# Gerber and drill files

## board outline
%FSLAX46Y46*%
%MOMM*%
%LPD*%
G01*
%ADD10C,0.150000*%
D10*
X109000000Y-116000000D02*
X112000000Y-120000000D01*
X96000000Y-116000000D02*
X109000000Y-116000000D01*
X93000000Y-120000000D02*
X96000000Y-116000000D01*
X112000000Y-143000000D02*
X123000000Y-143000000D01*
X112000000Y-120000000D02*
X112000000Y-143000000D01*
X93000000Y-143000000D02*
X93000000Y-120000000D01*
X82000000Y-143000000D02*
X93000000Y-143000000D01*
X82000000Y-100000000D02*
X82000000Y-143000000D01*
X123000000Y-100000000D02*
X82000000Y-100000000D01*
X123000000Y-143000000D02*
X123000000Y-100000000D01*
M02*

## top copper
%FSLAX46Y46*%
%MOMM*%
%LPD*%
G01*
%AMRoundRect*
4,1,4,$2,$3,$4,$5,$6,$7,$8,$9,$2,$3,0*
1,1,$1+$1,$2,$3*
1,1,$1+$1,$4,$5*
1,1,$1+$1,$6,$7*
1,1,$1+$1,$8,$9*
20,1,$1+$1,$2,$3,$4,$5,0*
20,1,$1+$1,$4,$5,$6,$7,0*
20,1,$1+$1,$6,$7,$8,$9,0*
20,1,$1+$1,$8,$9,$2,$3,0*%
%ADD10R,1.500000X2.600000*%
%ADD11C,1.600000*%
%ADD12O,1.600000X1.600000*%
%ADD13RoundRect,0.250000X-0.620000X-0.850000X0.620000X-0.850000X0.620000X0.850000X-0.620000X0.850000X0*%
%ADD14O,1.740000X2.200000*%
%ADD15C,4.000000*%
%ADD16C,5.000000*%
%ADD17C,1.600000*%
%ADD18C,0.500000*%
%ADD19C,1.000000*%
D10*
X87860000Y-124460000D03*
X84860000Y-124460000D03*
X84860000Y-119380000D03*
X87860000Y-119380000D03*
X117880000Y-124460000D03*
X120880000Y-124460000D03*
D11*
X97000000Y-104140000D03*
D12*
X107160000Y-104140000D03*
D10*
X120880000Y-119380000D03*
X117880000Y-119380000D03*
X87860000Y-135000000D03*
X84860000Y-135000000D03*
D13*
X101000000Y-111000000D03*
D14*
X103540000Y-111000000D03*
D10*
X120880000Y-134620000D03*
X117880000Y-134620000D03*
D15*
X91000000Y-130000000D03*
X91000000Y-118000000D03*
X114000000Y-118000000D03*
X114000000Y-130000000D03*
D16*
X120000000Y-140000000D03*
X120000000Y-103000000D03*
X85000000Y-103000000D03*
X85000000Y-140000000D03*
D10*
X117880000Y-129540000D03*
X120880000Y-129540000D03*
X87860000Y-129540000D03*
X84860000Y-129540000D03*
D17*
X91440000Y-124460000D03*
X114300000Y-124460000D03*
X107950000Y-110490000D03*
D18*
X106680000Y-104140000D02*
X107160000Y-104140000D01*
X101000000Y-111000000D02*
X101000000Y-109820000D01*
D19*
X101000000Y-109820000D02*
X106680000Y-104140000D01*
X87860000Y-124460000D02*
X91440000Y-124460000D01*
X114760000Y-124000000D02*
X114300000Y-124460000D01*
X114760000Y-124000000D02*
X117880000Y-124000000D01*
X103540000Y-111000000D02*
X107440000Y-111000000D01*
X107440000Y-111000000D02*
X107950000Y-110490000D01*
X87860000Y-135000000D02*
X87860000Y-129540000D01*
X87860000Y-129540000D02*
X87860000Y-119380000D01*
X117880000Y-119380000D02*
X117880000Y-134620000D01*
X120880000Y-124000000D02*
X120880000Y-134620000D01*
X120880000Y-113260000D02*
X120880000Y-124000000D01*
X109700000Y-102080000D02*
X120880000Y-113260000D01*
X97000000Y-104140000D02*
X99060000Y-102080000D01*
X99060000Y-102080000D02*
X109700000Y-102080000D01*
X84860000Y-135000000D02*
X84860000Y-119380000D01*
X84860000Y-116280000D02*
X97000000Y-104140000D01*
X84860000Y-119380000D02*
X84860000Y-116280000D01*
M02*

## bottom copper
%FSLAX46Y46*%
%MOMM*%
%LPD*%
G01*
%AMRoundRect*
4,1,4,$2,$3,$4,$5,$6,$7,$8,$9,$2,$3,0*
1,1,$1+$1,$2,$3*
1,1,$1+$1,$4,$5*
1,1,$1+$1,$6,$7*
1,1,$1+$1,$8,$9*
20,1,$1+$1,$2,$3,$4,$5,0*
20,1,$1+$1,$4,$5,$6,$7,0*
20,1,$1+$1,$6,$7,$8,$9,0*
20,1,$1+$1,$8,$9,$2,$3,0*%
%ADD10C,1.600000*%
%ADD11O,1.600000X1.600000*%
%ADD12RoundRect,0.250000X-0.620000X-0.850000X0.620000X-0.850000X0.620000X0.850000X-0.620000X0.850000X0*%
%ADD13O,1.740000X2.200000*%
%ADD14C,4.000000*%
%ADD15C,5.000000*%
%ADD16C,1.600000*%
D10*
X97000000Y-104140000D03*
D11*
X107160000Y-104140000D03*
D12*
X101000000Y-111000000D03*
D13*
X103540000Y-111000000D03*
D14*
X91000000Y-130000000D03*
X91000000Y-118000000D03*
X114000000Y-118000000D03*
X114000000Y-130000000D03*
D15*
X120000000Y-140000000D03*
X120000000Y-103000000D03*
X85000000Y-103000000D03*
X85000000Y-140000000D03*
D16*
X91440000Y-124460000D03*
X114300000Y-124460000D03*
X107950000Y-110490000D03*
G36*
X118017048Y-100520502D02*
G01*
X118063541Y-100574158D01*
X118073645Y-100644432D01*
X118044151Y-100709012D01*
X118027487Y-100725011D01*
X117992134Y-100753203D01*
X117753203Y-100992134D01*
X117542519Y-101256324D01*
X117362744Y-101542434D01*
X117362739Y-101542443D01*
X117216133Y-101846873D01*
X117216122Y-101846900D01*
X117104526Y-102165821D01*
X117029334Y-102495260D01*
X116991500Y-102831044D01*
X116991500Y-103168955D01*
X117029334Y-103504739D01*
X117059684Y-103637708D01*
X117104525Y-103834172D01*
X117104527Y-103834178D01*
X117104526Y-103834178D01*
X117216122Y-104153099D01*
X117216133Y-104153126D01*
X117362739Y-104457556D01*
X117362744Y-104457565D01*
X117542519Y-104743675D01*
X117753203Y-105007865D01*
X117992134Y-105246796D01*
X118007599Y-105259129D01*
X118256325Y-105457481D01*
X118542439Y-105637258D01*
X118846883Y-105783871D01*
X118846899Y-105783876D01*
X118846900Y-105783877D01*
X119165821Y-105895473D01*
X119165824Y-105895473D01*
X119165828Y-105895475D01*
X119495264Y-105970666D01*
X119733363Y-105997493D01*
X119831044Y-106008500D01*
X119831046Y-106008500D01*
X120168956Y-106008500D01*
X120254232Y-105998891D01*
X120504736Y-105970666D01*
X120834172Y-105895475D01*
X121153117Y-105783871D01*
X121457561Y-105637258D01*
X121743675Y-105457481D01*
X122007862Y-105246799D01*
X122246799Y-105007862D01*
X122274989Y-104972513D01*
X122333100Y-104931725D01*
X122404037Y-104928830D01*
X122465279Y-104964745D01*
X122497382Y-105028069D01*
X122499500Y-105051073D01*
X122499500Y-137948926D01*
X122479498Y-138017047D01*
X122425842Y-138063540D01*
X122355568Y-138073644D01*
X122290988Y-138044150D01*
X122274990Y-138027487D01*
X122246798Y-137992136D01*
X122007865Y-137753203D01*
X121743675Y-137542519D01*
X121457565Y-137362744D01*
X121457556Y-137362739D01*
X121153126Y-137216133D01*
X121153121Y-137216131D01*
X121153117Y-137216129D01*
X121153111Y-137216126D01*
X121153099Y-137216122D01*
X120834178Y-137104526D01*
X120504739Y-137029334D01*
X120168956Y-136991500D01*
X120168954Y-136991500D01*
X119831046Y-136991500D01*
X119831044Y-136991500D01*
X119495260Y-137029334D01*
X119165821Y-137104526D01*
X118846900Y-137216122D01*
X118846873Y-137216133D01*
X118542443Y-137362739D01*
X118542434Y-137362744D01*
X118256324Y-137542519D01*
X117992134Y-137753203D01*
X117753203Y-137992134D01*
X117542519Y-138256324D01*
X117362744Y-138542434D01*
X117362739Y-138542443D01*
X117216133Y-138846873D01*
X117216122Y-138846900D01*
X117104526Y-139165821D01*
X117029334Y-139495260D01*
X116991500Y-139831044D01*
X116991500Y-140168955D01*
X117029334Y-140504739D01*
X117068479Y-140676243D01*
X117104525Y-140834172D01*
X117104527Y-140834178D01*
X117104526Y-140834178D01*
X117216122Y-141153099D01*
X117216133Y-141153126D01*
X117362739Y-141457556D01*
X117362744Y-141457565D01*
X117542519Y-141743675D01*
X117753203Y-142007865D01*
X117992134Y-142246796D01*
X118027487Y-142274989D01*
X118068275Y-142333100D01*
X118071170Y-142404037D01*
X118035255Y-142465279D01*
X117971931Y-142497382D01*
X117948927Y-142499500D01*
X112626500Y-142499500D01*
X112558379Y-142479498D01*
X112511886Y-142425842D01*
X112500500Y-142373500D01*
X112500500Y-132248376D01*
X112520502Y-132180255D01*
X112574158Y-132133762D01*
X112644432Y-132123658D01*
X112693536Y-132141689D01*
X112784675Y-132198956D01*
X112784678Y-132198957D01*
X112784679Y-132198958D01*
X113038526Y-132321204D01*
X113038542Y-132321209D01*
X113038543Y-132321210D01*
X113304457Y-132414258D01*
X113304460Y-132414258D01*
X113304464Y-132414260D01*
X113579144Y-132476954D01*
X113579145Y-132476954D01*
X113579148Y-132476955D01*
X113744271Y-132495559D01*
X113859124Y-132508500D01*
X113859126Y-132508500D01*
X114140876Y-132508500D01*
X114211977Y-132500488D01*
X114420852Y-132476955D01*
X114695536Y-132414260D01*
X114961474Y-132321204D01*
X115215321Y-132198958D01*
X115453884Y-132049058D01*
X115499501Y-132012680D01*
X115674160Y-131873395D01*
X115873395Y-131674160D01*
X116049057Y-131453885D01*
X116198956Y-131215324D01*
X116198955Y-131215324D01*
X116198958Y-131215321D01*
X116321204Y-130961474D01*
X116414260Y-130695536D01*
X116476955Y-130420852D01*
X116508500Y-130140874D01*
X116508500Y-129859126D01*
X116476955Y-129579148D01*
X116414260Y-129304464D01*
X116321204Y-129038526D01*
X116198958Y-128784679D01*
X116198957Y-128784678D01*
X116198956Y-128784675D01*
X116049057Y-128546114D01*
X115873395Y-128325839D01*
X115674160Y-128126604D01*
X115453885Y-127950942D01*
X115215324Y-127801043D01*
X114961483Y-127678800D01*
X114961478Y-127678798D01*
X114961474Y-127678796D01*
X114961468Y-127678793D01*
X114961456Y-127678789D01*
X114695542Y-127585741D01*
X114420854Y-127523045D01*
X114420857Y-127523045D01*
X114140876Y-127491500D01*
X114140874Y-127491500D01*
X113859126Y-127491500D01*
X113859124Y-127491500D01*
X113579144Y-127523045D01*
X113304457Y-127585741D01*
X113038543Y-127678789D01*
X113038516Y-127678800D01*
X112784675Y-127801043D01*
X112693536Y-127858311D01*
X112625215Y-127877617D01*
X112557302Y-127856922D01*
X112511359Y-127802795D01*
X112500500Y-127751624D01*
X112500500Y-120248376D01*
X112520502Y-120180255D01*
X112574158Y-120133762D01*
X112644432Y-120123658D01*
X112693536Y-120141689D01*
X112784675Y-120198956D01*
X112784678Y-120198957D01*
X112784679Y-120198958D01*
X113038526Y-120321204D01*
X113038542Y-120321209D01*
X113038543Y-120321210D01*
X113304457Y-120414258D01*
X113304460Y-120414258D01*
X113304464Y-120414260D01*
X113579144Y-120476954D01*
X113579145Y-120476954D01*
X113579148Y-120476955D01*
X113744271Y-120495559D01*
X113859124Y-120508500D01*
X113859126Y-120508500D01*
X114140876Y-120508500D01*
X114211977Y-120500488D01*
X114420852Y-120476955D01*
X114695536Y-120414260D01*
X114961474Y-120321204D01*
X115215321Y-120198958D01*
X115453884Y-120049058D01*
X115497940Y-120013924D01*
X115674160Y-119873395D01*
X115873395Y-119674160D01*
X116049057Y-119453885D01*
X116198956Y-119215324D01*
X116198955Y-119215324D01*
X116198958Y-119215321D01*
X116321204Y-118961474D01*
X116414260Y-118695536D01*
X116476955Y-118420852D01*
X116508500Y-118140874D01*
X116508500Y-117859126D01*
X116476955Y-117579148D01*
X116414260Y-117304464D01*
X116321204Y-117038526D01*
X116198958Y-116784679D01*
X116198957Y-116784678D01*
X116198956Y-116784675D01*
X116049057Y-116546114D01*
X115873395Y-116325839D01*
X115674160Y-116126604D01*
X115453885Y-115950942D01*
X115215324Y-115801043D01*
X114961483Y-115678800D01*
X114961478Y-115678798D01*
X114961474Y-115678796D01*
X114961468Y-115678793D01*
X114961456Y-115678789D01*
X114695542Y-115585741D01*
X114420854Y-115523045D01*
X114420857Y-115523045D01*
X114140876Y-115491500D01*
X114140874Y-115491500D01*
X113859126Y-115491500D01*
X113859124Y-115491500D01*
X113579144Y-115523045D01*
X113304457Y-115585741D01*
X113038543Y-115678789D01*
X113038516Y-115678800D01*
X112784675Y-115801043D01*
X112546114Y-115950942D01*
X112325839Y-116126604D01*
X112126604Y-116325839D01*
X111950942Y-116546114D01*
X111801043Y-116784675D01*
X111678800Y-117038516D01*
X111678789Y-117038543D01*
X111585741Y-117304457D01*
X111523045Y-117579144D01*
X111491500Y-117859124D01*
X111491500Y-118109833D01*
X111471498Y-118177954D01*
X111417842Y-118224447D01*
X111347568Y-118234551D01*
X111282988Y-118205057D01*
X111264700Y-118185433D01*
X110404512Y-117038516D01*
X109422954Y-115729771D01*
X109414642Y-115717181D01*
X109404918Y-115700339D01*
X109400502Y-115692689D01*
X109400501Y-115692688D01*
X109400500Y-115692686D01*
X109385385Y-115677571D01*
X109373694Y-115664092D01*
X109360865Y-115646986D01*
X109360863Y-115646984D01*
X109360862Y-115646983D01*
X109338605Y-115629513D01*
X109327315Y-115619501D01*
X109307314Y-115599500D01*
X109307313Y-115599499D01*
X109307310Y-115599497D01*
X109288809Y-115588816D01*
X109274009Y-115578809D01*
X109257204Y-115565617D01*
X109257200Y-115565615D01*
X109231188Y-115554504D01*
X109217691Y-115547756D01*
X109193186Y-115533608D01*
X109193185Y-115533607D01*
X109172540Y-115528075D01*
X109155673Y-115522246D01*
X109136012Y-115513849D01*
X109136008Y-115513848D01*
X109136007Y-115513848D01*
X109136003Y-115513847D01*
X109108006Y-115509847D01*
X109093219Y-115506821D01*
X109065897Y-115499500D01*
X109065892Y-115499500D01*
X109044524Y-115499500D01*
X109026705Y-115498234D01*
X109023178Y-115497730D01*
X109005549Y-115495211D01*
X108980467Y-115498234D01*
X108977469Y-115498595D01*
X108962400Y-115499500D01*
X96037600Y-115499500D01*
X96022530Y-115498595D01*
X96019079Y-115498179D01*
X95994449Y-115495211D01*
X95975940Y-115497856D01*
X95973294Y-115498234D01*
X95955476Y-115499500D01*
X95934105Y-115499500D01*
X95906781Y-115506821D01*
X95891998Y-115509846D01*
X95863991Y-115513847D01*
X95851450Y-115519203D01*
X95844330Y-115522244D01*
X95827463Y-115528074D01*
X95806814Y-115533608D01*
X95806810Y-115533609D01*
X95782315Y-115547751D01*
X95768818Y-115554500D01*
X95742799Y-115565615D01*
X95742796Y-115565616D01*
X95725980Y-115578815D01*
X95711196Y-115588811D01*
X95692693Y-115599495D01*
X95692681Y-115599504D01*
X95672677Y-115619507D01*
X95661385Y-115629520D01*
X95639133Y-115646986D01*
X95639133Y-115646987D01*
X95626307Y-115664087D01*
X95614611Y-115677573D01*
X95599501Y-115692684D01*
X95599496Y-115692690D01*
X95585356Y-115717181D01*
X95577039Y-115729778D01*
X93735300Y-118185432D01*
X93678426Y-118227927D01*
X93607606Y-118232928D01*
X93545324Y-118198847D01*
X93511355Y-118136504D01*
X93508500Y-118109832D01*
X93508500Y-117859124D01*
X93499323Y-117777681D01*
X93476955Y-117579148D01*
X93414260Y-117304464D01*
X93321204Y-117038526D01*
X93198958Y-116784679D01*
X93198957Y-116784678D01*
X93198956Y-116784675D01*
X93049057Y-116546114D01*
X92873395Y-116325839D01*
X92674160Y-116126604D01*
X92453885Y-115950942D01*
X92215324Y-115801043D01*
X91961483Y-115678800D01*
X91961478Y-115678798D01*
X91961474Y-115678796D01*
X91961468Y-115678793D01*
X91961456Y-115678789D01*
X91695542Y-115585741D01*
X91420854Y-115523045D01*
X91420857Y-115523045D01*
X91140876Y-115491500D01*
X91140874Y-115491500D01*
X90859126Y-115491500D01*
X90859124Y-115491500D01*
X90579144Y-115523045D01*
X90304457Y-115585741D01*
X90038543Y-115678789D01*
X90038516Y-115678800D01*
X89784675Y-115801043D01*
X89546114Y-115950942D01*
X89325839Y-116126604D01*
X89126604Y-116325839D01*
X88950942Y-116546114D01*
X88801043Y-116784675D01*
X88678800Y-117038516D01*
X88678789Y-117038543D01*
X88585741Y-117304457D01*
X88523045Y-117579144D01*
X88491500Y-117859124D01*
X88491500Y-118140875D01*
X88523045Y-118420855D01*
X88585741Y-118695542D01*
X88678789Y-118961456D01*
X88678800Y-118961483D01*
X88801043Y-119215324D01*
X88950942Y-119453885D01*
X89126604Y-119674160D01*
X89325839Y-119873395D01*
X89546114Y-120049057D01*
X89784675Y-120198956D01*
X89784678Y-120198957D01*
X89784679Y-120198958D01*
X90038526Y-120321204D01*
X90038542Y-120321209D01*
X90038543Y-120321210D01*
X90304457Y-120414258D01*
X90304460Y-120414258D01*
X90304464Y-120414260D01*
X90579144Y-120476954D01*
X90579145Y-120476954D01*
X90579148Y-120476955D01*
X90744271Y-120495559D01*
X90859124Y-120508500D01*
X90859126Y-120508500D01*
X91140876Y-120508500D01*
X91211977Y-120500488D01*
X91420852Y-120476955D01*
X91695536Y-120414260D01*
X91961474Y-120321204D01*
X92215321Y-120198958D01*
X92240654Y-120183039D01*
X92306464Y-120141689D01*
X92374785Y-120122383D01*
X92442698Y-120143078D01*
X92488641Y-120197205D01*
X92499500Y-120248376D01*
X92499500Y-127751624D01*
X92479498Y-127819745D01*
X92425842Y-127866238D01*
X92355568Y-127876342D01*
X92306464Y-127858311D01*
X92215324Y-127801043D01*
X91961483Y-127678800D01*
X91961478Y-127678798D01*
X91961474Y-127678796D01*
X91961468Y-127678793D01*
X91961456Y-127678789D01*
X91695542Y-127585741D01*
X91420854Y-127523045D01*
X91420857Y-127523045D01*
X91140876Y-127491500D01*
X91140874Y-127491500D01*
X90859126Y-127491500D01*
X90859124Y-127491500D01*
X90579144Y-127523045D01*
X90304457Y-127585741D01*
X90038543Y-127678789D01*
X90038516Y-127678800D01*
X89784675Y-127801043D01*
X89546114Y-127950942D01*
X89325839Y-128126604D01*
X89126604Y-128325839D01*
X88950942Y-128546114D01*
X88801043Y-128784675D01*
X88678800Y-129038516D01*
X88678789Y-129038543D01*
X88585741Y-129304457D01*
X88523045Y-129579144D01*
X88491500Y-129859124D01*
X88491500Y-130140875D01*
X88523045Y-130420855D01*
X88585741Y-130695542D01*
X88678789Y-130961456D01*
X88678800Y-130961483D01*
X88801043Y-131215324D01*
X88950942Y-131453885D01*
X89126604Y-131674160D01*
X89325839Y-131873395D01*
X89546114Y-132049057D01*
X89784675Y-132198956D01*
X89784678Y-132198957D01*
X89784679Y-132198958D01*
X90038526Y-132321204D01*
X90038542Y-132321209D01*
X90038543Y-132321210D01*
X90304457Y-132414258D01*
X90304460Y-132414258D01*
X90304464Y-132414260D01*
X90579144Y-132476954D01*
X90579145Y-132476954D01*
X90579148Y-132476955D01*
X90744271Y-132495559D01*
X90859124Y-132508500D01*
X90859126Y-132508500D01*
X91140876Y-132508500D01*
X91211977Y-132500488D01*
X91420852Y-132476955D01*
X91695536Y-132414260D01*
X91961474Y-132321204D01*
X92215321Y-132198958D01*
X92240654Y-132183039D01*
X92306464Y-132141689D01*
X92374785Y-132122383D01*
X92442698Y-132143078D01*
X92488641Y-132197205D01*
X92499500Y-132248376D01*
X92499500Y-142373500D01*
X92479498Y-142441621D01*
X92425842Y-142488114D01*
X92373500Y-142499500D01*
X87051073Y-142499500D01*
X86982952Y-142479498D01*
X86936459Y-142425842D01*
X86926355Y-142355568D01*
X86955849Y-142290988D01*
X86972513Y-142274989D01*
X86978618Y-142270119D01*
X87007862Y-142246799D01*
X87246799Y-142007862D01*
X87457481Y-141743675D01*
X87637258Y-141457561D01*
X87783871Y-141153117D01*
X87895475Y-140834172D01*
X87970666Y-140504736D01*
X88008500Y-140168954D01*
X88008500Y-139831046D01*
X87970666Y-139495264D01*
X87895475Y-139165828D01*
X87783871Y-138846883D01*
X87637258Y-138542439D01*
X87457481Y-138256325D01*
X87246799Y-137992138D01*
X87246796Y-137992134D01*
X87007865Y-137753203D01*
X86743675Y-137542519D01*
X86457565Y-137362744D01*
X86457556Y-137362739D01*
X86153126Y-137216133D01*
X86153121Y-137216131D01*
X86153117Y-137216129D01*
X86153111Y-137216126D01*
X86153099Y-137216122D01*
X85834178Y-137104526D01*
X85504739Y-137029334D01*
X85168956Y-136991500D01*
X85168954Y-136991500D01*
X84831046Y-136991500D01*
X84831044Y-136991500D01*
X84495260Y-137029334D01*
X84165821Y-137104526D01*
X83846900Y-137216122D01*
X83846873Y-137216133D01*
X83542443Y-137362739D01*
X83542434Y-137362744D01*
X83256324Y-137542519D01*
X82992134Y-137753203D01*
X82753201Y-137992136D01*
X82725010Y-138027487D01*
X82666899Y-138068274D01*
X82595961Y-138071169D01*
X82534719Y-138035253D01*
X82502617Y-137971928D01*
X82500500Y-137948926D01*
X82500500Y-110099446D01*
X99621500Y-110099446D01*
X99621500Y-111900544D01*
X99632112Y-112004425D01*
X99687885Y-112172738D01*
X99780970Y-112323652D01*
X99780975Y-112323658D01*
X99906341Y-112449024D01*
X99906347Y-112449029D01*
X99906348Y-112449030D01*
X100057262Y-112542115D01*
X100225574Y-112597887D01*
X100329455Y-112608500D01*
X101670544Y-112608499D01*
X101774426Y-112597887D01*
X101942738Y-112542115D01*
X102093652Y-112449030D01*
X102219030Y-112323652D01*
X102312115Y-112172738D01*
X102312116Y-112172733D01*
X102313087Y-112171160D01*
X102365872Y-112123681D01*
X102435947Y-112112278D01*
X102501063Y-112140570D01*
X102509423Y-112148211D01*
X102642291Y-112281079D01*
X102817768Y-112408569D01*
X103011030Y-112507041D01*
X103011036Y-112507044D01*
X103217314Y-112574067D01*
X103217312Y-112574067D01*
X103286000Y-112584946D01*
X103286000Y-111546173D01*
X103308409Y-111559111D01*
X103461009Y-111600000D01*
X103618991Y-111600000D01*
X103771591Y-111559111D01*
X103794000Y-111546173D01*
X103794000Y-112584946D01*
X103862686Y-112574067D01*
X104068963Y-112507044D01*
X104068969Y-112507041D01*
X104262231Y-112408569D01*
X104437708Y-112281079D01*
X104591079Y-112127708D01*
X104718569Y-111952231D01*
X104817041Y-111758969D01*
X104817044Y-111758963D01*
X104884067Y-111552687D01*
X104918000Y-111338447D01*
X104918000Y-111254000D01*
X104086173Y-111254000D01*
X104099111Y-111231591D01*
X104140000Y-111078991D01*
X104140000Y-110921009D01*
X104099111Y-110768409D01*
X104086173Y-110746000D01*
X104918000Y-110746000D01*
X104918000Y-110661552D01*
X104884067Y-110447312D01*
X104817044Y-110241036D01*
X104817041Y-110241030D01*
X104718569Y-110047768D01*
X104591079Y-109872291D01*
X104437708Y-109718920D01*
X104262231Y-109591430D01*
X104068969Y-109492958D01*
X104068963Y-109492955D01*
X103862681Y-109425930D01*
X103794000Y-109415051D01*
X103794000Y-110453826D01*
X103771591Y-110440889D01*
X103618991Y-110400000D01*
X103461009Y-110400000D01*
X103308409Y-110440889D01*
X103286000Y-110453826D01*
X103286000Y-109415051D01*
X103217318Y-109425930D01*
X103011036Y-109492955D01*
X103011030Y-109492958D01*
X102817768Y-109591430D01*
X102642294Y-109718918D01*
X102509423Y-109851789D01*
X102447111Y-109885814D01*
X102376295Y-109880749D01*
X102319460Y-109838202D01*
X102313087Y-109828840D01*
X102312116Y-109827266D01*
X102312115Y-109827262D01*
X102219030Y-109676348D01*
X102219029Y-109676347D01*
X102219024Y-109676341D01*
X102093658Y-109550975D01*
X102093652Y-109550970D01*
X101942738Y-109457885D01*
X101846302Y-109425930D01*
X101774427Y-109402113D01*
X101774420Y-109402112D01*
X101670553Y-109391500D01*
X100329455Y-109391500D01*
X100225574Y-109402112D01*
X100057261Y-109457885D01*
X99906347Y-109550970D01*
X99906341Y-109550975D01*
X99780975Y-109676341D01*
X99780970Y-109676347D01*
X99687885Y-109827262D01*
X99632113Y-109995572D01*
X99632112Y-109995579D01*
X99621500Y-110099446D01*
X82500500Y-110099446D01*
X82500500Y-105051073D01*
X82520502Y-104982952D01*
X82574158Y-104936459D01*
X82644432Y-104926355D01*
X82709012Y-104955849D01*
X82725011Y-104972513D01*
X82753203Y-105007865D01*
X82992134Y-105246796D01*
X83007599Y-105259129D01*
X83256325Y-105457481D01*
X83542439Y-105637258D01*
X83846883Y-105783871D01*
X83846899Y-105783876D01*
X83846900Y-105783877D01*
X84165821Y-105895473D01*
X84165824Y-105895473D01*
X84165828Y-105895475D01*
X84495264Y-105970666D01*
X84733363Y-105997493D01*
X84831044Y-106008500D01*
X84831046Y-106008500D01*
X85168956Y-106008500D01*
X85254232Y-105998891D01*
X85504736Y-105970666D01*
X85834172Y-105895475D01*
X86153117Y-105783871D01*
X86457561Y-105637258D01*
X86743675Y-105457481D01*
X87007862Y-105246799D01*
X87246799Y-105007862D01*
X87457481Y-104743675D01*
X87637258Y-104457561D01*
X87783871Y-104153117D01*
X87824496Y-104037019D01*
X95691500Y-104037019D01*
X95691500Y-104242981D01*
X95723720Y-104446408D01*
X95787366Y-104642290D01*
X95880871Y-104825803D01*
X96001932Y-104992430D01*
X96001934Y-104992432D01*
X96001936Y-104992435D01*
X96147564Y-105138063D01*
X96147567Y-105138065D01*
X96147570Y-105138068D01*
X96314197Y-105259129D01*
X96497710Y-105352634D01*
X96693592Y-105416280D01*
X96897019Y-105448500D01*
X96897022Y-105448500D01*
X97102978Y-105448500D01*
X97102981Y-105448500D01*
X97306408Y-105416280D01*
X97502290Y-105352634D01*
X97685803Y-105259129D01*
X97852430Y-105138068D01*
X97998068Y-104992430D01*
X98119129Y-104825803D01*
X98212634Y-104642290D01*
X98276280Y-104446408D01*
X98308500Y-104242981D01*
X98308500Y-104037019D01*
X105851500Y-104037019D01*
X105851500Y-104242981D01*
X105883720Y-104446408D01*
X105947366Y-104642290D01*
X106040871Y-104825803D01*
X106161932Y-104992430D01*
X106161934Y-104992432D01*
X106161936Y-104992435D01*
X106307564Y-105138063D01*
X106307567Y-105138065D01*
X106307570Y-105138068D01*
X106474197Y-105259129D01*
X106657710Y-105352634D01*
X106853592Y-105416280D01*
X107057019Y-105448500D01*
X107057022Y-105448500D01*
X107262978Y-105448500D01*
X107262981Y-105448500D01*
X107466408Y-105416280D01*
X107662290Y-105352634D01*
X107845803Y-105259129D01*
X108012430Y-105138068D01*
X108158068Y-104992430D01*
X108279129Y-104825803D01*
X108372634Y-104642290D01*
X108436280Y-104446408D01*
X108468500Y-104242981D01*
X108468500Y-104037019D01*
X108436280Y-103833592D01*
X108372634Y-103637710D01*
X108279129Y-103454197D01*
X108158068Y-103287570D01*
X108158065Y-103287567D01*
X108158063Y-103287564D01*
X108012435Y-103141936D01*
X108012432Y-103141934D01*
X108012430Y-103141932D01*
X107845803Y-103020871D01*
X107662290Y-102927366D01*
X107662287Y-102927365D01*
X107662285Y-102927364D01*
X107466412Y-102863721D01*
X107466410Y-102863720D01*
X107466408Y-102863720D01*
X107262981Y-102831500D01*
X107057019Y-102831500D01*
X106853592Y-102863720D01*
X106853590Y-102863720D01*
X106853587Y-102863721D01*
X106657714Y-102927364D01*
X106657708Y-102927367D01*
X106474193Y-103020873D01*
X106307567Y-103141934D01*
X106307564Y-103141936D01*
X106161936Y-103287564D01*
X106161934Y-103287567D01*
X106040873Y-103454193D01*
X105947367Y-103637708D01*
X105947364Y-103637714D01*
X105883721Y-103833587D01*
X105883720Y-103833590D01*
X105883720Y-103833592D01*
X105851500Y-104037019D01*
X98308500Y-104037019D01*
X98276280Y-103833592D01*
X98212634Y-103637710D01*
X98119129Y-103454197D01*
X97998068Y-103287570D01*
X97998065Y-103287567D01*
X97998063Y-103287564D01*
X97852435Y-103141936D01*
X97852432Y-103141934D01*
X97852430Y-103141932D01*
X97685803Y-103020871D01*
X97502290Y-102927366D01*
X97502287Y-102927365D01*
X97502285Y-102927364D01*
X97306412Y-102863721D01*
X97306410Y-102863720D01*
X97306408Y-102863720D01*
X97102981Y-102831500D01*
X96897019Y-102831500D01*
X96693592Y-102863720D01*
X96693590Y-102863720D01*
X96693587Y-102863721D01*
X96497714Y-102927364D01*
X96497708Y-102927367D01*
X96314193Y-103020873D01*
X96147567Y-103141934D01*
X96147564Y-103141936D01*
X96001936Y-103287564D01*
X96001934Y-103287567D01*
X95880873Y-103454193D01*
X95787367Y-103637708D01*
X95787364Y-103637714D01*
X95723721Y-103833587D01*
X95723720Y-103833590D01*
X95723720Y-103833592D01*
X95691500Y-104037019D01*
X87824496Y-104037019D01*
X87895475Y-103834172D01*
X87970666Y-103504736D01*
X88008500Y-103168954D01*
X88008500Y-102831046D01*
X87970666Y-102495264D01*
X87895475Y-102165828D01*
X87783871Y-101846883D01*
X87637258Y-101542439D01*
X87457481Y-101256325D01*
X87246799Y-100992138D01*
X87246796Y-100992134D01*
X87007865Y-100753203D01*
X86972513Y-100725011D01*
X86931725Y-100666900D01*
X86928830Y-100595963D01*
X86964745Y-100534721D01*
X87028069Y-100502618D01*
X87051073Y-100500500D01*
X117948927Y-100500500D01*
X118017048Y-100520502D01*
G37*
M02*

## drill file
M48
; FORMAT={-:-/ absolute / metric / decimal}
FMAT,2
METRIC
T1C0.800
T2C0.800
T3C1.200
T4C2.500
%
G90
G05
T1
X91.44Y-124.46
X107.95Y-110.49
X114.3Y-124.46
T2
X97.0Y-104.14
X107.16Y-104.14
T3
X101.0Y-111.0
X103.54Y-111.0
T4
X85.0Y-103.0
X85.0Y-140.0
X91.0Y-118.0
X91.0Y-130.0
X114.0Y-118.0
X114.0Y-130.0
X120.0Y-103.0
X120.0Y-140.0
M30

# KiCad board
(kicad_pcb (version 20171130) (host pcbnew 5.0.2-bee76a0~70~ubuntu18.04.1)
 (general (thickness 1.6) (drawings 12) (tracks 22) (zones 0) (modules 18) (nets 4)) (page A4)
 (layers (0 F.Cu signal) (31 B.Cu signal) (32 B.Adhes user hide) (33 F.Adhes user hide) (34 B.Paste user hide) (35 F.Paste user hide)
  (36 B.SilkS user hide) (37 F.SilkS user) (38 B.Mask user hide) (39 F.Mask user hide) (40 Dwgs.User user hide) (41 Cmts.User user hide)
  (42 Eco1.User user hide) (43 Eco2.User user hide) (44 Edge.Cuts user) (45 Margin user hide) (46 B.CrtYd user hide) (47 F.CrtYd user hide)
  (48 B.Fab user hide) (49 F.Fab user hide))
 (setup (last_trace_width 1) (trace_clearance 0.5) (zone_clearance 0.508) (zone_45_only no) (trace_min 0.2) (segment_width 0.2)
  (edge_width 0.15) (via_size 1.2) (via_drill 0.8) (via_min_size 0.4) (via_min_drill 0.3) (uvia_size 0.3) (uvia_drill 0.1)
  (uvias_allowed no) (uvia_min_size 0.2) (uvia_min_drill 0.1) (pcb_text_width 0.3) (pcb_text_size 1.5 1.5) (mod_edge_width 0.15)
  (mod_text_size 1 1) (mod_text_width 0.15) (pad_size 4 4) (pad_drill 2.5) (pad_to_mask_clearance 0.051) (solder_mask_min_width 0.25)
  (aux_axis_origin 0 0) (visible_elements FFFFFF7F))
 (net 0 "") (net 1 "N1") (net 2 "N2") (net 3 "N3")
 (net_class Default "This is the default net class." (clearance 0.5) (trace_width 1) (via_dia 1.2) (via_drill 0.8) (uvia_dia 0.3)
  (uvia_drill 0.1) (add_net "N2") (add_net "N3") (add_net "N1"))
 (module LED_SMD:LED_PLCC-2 (layer F.Cu) (at 86.36 124.46 180)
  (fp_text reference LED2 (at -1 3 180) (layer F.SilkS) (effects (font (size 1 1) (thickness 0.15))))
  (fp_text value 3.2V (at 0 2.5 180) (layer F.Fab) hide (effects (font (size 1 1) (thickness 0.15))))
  (pad 1 smd rect (at -1.5 0 180) (size 1.5 2.6) (layers F.Cu F.Paste F.Mask) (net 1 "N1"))
  (pad 2 smd rect (at 1.5 0 180) (size 1.5 2.6) (layers F.Cu F.Paste F.Mask) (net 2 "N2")))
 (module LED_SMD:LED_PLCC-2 (layer F.Cu) (at 86.36 119.38 180)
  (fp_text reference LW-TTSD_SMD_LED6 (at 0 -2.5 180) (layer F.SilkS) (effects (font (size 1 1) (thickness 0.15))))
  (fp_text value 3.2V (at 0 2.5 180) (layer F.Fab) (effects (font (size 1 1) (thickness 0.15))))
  (pad 2 smd rect (at 1.5 0 180) (size 1.5 2.6) (layers F.Cu F.Paste F.Mask) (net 2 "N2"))
  (pad 1 smd rect (at -1.5 0 180) (size 1.5 2.6) (layers F.Cu F.Paste F.Mask) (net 1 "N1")))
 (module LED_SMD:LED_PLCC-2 (layer F.Cu) (at 119.38 124.46)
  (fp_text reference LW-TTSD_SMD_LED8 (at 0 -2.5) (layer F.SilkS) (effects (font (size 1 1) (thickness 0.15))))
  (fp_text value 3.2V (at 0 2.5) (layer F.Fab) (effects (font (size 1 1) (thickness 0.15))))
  (pad 1 smd rect (at -1.5 0) (size 1.5 2.6) (layers F.Cu F.Paste F.Mask) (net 1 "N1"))
  (pad 2 smd rect (at 1.5 0) (size 1.5 2.6) (layers F.Cu F.Paste F.Mask) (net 2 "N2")))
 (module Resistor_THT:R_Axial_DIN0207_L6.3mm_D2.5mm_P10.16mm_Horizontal (layer F.Cu) (at 97 104.14)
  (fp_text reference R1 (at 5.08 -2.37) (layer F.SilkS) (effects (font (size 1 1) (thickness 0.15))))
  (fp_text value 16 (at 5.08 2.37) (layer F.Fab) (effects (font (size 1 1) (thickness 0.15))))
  (pad 1 thru_hole circle (at 0 0) (size 1.6 1.6) (drill 0.8) (layers *.Cu *.Mask) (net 2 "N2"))
  (pad 2 thru_hole oval (at 10.16 0) (size 1.6 1.6) (drill 0.8) (layers *.Cu *.Mask) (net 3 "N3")))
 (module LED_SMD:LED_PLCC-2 (layer F.Cu) (at 119.38 119.38)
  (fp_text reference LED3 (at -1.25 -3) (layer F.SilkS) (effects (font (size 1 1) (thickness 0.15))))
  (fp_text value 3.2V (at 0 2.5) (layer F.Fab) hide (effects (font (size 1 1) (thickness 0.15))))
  (pad 2 smd rect (at 1.5 0) (size 1.5 2.6) (layers F.Cu F.Paste F.Mask) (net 2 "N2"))
  (pad 1 smd rect (at -1.5 0) (size 1.5 2.6) (layers F.Cu F.Paste F.Mask) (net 1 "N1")))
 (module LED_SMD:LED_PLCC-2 (layer F.Cu) (at 86.36 135 180)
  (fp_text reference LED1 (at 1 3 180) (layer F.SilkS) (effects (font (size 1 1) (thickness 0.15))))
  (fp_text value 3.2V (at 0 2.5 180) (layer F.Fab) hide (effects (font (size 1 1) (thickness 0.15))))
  (pad 1 smd rect (at -1.5 0 180) (size 1.5 2.6) (layers F.Cu F.Paste F.Mask) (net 1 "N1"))
  (pad 2 smd rect (at 1.5 0 180) (size 1.5 2.6) (layers F.Cu F.Paste F.Mask) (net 2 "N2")))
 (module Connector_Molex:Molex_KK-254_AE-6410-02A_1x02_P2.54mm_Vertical (layer B.Cu) (at 101 111)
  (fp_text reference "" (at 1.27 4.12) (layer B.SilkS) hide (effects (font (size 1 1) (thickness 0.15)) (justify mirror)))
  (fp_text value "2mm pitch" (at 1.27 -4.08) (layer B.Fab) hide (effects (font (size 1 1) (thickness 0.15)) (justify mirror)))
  (pad 1 thru_hole roundrect (at 0 0) (size 1.74 2.2) (drill 1.2) (layers *.Cu *.Mask) (roundrect_rratio 0.143678) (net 3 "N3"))
  (pad 2 thru_hole oval (at 2.54 0) (size 1.74 2.2) (drill 1.2) (layers *.Cu *.Mask) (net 1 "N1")))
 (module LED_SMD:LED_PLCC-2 (layer F.Cu) (at 119.38 134.62)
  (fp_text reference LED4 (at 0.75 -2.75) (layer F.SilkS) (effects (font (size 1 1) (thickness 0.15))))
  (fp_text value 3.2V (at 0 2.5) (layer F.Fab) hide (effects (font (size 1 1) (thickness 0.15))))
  (pad 2 smd rect (at 1.5 0) (size 1.5 2.6) (layers F.Cu F.Paste F.Mask) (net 2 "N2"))
  (pad 1 smd rect (at -1.5 0) (size 1.5 2.6) (layers F.Cu F.Paste F.Mask) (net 1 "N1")))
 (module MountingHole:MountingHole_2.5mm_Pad (layer F.Cu) (at 91 130)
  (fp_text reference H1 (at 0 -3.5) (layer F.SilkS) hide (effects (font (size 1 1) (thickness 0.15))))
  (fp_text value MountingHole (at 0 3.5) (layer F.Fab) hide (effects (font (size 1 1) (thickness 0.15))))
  (pad 1 thru_hole circle (at 0 0) (size 4 4) (drill 2.5) (layers *.Cu *.Mask)))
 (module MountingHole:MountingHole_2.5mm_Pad (layer F.Cu) (at 91 118)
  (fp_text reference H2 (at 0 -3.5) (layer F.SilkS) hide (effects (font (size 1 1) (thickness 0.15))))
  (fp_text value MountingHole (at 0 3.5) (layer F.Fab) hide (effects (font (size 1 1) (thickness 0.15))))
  (pad 1 thru_hole circle (at 0 0) (size 4 4) (drill 2.5) (layers *.Cu *.Mask)))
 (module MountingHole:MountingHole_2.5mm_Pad (layer F.Cu) (at 114 118)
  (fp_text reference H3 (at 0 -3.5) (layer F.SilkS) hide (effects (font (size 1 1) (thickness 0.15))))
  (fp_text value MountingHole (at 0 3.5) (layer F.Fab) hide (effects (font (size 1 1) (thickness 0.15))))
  (pad 1 thru_hole circle (at 0 0) (size 4 4) (drill 2.5) (layers *.Cu *.Mask)))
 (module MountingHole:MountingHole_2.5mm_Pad (layer F.Cu) (at 114 130)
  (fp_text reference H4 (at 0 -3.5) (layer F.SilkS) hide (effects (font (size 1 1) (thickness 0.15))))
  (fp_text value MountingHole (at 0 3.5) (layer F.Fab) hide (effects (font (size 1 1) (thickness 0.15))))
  (pad 1 thru_hole circle (at 0 0) (size 4 4) (drill 2.5) (layers *.Cu *.Mask)))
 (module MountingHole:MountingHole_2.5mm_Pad (layer F.Cu) (at 120 140)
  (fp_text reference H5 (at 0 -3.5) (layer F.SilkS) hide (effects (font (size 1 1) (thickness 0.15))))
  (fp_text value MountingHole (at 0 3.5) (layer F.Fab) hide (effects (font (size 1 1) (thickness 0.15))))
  (pad 1 thru_hole circle (at 0 0) (size 5 5) (drill 2.5) (layers *.Cu *.Mask)))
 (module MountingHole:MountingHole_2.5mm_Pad (layer F.Cu) (at 120 103)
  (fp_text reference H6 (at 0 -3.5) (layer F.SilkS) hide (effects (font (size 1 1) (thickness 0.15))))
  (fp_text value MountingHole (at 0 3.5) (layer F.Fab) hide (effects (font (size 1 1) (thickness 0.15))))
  (pad 1 thru_hole circle (at 0 0) (size 5 5) (drill 2.5) (layers *.Cu *.Mask)))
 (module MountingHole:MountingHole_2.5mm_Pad (layer F.Cu) (at 85 103)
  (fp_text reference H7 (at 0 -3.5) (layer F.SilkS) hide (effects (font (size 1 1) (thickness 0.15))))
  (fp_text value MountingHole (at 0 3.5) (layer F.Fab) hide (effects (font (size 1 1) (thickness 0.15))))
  (pad 1 thru_hole circle (at 0 0) (size 5 5) (drill 2.5) (layers *.Cu *.Mask)))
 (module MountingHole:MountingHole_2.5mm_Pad (layer F.Cu) (at 85 140)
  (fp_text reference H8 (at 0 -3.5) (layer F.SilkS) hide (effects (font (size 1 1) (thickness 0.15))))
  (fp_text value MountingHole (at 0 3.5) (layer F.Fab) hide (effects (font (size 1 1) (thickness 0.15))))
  (pad 1 thru_hole circle (at 0 0) (size 5 5) (drill 2.5) (layers *.Cu *.Mask)))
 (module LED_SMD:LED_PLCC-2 (layer F.Cu) (at 119.38 129.54)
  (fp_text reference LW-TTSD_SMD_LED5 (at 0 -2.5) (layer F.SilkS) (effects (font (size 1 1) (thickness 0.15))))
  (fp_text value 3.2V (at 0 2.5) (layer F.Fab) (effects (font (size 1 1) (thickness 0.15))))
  (pad 1 smd rect (at -1.5 0) (size 1.5 2.6) (layers F.Cu F.Paste F.Mask) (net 1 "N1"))
  (pad 2 smd rect (at 1.5 0) (size 1.5 2.6) (layers F.Cu F.Paste F.Mask) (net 2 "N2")))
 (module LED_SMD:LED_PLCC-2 (layer F.Cu) (at 86.36 129.54 180)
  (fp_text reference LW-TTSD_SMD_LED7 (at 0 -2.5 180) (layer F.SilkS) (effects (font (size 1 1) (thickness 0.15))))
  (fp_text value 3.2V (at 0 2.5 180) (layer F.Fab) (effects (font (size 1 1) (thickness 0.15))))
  (pad 1 smd rect (at -1.5 0 180) (size 1.5 2.6) (layers F.Cu F.Paste F.Mask) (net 1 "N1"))
  (pad 2 smd rect (at 1.5 0 180) (size 1.5 2.6) (layers F.Cu F.Paste F.Mask) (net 2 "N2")))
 (gr_line (start 109 116) (end 112 120) (layer Edge.Cuts) (width 0.15))
 (gr_line (start 96 116) (end 109 116) (layer Edge.Cuts) (width 0.15))
 (gr_line (start 93 120) (end 96 116) (layer Edge.Cuts) (width 0.15))
 (gr_line (start 112 143) (end 123 143) (layer Edge.Cuts) (width 0.15))
 (gr_line (start 112 120) (end 112 143) (layer Edge.Cuts) (width 0.15))
 (gr_line (start 93 143) (end 93 120) (layer Edge.Cuts) (width 0.15))
 (gr_line (start 82 143) (end 93 143) (layer Edge.Cuts) (width 0.15))
 (gr_line (start 82 100) (end 82 143) (layer Edge.Cuts) (width 0.15))
 (gr_line (start 123 100) (end 82 100) (layer Edge.Cuts) (width 0.15))
 (gr_line (start 123 143) (end 123 100) (layer Edge.Cuts) (width 0.15))
 (segment (start 106.68 104.14) (end 107.16 104.14) (width 0.5) (layer F.Cu) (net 3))
 (segment (start 101 111) (end 101 109.82) (width 0.5) (layer F.Cu) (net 3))
 (segment (start 101 109.82) (end 106.68 104.14) (width 1) (layer F.Cu) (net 3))
 (via (at 91.44 124.46) (size 1.6) (drill 0.8) (layers F.Cu B.Cu) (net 1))
 (segment (start 87.86 124.46) (end 91.44 124.46) (width 1) (layer F.Cu) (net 1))
 (via (at 114.3 124.46) (size 1.6) (drill 0.8) (layers F.Cu B.Cu) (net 1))
 (segment (start 114.76 124) (end 114.3 124.46) (width 1) (layer F.Cu) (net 1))
 (segment (start 114.76 124) (end 117.88 124) (width 1) (layer F.Cu) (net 1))
 (via (at 107.95 110.49) (size 1.6) (drill 0.8) (layers F.Cu B.Cu) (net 1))
 (segment (start 103.54 111) (end 107.44 111) (width 1) (layer F.Cu) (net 1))
 (segment (start 107.44 111) (end 107.95 110.49) (width 1) (layer F.Cu) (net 1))
 (segment (start 87.86 135) (end 87.86 129.54) (width 1) (layer F.Cu) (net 1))
 (segment (start 87.86 129.54) (end 87.86 119.38) (width 1) (layer F.Cu) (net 1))
 (segment (start 117.88 119.38) (end 117.88 134.62) (width 1) (layer F.Cu) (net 1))
 (segment (start 120.88 124) (end 120.88 134.62) (width 1) (layer F.Cu) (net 2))
 (segment (start 120.88 113.26) (end 120.88 124) (width 1) (layer F.Cu) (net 2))
 (segment (start 109.7 102.08) (end 120.88 113.26) (width 1) (layer F.Cu) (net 2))
 (segment (start 97 104.14) (end 99.06 102.08) (width 1) (layer F.Cu) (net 2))
 (segment (start 99.06 102.08) (end 109.7 102.08) (width 1) (layer F.Cu) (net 2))
 (segment (start 84.86 135) (end 84.86 119.38) (width 1) (layer F.Cu) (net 2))
 (segment (start 84.86 116.28) (end 97 104.14) (width 1) (layer F.Cu) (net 2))
 (segment (start 84.86 119.38) (end 84.86 116.28) (width 1) (layer F.Cu) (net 2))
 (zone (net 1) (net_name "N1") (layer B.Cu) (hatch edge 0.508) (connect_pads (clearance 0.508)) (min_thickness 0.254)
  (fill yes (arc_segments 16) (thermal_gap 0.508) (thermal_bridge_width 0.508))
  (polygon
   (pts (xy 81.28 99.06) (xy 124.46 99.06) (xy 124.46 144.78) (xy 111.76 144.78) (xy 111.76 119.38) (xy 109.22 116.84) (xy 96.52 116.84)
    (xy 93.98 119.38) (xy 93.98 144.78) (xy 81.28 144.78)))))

